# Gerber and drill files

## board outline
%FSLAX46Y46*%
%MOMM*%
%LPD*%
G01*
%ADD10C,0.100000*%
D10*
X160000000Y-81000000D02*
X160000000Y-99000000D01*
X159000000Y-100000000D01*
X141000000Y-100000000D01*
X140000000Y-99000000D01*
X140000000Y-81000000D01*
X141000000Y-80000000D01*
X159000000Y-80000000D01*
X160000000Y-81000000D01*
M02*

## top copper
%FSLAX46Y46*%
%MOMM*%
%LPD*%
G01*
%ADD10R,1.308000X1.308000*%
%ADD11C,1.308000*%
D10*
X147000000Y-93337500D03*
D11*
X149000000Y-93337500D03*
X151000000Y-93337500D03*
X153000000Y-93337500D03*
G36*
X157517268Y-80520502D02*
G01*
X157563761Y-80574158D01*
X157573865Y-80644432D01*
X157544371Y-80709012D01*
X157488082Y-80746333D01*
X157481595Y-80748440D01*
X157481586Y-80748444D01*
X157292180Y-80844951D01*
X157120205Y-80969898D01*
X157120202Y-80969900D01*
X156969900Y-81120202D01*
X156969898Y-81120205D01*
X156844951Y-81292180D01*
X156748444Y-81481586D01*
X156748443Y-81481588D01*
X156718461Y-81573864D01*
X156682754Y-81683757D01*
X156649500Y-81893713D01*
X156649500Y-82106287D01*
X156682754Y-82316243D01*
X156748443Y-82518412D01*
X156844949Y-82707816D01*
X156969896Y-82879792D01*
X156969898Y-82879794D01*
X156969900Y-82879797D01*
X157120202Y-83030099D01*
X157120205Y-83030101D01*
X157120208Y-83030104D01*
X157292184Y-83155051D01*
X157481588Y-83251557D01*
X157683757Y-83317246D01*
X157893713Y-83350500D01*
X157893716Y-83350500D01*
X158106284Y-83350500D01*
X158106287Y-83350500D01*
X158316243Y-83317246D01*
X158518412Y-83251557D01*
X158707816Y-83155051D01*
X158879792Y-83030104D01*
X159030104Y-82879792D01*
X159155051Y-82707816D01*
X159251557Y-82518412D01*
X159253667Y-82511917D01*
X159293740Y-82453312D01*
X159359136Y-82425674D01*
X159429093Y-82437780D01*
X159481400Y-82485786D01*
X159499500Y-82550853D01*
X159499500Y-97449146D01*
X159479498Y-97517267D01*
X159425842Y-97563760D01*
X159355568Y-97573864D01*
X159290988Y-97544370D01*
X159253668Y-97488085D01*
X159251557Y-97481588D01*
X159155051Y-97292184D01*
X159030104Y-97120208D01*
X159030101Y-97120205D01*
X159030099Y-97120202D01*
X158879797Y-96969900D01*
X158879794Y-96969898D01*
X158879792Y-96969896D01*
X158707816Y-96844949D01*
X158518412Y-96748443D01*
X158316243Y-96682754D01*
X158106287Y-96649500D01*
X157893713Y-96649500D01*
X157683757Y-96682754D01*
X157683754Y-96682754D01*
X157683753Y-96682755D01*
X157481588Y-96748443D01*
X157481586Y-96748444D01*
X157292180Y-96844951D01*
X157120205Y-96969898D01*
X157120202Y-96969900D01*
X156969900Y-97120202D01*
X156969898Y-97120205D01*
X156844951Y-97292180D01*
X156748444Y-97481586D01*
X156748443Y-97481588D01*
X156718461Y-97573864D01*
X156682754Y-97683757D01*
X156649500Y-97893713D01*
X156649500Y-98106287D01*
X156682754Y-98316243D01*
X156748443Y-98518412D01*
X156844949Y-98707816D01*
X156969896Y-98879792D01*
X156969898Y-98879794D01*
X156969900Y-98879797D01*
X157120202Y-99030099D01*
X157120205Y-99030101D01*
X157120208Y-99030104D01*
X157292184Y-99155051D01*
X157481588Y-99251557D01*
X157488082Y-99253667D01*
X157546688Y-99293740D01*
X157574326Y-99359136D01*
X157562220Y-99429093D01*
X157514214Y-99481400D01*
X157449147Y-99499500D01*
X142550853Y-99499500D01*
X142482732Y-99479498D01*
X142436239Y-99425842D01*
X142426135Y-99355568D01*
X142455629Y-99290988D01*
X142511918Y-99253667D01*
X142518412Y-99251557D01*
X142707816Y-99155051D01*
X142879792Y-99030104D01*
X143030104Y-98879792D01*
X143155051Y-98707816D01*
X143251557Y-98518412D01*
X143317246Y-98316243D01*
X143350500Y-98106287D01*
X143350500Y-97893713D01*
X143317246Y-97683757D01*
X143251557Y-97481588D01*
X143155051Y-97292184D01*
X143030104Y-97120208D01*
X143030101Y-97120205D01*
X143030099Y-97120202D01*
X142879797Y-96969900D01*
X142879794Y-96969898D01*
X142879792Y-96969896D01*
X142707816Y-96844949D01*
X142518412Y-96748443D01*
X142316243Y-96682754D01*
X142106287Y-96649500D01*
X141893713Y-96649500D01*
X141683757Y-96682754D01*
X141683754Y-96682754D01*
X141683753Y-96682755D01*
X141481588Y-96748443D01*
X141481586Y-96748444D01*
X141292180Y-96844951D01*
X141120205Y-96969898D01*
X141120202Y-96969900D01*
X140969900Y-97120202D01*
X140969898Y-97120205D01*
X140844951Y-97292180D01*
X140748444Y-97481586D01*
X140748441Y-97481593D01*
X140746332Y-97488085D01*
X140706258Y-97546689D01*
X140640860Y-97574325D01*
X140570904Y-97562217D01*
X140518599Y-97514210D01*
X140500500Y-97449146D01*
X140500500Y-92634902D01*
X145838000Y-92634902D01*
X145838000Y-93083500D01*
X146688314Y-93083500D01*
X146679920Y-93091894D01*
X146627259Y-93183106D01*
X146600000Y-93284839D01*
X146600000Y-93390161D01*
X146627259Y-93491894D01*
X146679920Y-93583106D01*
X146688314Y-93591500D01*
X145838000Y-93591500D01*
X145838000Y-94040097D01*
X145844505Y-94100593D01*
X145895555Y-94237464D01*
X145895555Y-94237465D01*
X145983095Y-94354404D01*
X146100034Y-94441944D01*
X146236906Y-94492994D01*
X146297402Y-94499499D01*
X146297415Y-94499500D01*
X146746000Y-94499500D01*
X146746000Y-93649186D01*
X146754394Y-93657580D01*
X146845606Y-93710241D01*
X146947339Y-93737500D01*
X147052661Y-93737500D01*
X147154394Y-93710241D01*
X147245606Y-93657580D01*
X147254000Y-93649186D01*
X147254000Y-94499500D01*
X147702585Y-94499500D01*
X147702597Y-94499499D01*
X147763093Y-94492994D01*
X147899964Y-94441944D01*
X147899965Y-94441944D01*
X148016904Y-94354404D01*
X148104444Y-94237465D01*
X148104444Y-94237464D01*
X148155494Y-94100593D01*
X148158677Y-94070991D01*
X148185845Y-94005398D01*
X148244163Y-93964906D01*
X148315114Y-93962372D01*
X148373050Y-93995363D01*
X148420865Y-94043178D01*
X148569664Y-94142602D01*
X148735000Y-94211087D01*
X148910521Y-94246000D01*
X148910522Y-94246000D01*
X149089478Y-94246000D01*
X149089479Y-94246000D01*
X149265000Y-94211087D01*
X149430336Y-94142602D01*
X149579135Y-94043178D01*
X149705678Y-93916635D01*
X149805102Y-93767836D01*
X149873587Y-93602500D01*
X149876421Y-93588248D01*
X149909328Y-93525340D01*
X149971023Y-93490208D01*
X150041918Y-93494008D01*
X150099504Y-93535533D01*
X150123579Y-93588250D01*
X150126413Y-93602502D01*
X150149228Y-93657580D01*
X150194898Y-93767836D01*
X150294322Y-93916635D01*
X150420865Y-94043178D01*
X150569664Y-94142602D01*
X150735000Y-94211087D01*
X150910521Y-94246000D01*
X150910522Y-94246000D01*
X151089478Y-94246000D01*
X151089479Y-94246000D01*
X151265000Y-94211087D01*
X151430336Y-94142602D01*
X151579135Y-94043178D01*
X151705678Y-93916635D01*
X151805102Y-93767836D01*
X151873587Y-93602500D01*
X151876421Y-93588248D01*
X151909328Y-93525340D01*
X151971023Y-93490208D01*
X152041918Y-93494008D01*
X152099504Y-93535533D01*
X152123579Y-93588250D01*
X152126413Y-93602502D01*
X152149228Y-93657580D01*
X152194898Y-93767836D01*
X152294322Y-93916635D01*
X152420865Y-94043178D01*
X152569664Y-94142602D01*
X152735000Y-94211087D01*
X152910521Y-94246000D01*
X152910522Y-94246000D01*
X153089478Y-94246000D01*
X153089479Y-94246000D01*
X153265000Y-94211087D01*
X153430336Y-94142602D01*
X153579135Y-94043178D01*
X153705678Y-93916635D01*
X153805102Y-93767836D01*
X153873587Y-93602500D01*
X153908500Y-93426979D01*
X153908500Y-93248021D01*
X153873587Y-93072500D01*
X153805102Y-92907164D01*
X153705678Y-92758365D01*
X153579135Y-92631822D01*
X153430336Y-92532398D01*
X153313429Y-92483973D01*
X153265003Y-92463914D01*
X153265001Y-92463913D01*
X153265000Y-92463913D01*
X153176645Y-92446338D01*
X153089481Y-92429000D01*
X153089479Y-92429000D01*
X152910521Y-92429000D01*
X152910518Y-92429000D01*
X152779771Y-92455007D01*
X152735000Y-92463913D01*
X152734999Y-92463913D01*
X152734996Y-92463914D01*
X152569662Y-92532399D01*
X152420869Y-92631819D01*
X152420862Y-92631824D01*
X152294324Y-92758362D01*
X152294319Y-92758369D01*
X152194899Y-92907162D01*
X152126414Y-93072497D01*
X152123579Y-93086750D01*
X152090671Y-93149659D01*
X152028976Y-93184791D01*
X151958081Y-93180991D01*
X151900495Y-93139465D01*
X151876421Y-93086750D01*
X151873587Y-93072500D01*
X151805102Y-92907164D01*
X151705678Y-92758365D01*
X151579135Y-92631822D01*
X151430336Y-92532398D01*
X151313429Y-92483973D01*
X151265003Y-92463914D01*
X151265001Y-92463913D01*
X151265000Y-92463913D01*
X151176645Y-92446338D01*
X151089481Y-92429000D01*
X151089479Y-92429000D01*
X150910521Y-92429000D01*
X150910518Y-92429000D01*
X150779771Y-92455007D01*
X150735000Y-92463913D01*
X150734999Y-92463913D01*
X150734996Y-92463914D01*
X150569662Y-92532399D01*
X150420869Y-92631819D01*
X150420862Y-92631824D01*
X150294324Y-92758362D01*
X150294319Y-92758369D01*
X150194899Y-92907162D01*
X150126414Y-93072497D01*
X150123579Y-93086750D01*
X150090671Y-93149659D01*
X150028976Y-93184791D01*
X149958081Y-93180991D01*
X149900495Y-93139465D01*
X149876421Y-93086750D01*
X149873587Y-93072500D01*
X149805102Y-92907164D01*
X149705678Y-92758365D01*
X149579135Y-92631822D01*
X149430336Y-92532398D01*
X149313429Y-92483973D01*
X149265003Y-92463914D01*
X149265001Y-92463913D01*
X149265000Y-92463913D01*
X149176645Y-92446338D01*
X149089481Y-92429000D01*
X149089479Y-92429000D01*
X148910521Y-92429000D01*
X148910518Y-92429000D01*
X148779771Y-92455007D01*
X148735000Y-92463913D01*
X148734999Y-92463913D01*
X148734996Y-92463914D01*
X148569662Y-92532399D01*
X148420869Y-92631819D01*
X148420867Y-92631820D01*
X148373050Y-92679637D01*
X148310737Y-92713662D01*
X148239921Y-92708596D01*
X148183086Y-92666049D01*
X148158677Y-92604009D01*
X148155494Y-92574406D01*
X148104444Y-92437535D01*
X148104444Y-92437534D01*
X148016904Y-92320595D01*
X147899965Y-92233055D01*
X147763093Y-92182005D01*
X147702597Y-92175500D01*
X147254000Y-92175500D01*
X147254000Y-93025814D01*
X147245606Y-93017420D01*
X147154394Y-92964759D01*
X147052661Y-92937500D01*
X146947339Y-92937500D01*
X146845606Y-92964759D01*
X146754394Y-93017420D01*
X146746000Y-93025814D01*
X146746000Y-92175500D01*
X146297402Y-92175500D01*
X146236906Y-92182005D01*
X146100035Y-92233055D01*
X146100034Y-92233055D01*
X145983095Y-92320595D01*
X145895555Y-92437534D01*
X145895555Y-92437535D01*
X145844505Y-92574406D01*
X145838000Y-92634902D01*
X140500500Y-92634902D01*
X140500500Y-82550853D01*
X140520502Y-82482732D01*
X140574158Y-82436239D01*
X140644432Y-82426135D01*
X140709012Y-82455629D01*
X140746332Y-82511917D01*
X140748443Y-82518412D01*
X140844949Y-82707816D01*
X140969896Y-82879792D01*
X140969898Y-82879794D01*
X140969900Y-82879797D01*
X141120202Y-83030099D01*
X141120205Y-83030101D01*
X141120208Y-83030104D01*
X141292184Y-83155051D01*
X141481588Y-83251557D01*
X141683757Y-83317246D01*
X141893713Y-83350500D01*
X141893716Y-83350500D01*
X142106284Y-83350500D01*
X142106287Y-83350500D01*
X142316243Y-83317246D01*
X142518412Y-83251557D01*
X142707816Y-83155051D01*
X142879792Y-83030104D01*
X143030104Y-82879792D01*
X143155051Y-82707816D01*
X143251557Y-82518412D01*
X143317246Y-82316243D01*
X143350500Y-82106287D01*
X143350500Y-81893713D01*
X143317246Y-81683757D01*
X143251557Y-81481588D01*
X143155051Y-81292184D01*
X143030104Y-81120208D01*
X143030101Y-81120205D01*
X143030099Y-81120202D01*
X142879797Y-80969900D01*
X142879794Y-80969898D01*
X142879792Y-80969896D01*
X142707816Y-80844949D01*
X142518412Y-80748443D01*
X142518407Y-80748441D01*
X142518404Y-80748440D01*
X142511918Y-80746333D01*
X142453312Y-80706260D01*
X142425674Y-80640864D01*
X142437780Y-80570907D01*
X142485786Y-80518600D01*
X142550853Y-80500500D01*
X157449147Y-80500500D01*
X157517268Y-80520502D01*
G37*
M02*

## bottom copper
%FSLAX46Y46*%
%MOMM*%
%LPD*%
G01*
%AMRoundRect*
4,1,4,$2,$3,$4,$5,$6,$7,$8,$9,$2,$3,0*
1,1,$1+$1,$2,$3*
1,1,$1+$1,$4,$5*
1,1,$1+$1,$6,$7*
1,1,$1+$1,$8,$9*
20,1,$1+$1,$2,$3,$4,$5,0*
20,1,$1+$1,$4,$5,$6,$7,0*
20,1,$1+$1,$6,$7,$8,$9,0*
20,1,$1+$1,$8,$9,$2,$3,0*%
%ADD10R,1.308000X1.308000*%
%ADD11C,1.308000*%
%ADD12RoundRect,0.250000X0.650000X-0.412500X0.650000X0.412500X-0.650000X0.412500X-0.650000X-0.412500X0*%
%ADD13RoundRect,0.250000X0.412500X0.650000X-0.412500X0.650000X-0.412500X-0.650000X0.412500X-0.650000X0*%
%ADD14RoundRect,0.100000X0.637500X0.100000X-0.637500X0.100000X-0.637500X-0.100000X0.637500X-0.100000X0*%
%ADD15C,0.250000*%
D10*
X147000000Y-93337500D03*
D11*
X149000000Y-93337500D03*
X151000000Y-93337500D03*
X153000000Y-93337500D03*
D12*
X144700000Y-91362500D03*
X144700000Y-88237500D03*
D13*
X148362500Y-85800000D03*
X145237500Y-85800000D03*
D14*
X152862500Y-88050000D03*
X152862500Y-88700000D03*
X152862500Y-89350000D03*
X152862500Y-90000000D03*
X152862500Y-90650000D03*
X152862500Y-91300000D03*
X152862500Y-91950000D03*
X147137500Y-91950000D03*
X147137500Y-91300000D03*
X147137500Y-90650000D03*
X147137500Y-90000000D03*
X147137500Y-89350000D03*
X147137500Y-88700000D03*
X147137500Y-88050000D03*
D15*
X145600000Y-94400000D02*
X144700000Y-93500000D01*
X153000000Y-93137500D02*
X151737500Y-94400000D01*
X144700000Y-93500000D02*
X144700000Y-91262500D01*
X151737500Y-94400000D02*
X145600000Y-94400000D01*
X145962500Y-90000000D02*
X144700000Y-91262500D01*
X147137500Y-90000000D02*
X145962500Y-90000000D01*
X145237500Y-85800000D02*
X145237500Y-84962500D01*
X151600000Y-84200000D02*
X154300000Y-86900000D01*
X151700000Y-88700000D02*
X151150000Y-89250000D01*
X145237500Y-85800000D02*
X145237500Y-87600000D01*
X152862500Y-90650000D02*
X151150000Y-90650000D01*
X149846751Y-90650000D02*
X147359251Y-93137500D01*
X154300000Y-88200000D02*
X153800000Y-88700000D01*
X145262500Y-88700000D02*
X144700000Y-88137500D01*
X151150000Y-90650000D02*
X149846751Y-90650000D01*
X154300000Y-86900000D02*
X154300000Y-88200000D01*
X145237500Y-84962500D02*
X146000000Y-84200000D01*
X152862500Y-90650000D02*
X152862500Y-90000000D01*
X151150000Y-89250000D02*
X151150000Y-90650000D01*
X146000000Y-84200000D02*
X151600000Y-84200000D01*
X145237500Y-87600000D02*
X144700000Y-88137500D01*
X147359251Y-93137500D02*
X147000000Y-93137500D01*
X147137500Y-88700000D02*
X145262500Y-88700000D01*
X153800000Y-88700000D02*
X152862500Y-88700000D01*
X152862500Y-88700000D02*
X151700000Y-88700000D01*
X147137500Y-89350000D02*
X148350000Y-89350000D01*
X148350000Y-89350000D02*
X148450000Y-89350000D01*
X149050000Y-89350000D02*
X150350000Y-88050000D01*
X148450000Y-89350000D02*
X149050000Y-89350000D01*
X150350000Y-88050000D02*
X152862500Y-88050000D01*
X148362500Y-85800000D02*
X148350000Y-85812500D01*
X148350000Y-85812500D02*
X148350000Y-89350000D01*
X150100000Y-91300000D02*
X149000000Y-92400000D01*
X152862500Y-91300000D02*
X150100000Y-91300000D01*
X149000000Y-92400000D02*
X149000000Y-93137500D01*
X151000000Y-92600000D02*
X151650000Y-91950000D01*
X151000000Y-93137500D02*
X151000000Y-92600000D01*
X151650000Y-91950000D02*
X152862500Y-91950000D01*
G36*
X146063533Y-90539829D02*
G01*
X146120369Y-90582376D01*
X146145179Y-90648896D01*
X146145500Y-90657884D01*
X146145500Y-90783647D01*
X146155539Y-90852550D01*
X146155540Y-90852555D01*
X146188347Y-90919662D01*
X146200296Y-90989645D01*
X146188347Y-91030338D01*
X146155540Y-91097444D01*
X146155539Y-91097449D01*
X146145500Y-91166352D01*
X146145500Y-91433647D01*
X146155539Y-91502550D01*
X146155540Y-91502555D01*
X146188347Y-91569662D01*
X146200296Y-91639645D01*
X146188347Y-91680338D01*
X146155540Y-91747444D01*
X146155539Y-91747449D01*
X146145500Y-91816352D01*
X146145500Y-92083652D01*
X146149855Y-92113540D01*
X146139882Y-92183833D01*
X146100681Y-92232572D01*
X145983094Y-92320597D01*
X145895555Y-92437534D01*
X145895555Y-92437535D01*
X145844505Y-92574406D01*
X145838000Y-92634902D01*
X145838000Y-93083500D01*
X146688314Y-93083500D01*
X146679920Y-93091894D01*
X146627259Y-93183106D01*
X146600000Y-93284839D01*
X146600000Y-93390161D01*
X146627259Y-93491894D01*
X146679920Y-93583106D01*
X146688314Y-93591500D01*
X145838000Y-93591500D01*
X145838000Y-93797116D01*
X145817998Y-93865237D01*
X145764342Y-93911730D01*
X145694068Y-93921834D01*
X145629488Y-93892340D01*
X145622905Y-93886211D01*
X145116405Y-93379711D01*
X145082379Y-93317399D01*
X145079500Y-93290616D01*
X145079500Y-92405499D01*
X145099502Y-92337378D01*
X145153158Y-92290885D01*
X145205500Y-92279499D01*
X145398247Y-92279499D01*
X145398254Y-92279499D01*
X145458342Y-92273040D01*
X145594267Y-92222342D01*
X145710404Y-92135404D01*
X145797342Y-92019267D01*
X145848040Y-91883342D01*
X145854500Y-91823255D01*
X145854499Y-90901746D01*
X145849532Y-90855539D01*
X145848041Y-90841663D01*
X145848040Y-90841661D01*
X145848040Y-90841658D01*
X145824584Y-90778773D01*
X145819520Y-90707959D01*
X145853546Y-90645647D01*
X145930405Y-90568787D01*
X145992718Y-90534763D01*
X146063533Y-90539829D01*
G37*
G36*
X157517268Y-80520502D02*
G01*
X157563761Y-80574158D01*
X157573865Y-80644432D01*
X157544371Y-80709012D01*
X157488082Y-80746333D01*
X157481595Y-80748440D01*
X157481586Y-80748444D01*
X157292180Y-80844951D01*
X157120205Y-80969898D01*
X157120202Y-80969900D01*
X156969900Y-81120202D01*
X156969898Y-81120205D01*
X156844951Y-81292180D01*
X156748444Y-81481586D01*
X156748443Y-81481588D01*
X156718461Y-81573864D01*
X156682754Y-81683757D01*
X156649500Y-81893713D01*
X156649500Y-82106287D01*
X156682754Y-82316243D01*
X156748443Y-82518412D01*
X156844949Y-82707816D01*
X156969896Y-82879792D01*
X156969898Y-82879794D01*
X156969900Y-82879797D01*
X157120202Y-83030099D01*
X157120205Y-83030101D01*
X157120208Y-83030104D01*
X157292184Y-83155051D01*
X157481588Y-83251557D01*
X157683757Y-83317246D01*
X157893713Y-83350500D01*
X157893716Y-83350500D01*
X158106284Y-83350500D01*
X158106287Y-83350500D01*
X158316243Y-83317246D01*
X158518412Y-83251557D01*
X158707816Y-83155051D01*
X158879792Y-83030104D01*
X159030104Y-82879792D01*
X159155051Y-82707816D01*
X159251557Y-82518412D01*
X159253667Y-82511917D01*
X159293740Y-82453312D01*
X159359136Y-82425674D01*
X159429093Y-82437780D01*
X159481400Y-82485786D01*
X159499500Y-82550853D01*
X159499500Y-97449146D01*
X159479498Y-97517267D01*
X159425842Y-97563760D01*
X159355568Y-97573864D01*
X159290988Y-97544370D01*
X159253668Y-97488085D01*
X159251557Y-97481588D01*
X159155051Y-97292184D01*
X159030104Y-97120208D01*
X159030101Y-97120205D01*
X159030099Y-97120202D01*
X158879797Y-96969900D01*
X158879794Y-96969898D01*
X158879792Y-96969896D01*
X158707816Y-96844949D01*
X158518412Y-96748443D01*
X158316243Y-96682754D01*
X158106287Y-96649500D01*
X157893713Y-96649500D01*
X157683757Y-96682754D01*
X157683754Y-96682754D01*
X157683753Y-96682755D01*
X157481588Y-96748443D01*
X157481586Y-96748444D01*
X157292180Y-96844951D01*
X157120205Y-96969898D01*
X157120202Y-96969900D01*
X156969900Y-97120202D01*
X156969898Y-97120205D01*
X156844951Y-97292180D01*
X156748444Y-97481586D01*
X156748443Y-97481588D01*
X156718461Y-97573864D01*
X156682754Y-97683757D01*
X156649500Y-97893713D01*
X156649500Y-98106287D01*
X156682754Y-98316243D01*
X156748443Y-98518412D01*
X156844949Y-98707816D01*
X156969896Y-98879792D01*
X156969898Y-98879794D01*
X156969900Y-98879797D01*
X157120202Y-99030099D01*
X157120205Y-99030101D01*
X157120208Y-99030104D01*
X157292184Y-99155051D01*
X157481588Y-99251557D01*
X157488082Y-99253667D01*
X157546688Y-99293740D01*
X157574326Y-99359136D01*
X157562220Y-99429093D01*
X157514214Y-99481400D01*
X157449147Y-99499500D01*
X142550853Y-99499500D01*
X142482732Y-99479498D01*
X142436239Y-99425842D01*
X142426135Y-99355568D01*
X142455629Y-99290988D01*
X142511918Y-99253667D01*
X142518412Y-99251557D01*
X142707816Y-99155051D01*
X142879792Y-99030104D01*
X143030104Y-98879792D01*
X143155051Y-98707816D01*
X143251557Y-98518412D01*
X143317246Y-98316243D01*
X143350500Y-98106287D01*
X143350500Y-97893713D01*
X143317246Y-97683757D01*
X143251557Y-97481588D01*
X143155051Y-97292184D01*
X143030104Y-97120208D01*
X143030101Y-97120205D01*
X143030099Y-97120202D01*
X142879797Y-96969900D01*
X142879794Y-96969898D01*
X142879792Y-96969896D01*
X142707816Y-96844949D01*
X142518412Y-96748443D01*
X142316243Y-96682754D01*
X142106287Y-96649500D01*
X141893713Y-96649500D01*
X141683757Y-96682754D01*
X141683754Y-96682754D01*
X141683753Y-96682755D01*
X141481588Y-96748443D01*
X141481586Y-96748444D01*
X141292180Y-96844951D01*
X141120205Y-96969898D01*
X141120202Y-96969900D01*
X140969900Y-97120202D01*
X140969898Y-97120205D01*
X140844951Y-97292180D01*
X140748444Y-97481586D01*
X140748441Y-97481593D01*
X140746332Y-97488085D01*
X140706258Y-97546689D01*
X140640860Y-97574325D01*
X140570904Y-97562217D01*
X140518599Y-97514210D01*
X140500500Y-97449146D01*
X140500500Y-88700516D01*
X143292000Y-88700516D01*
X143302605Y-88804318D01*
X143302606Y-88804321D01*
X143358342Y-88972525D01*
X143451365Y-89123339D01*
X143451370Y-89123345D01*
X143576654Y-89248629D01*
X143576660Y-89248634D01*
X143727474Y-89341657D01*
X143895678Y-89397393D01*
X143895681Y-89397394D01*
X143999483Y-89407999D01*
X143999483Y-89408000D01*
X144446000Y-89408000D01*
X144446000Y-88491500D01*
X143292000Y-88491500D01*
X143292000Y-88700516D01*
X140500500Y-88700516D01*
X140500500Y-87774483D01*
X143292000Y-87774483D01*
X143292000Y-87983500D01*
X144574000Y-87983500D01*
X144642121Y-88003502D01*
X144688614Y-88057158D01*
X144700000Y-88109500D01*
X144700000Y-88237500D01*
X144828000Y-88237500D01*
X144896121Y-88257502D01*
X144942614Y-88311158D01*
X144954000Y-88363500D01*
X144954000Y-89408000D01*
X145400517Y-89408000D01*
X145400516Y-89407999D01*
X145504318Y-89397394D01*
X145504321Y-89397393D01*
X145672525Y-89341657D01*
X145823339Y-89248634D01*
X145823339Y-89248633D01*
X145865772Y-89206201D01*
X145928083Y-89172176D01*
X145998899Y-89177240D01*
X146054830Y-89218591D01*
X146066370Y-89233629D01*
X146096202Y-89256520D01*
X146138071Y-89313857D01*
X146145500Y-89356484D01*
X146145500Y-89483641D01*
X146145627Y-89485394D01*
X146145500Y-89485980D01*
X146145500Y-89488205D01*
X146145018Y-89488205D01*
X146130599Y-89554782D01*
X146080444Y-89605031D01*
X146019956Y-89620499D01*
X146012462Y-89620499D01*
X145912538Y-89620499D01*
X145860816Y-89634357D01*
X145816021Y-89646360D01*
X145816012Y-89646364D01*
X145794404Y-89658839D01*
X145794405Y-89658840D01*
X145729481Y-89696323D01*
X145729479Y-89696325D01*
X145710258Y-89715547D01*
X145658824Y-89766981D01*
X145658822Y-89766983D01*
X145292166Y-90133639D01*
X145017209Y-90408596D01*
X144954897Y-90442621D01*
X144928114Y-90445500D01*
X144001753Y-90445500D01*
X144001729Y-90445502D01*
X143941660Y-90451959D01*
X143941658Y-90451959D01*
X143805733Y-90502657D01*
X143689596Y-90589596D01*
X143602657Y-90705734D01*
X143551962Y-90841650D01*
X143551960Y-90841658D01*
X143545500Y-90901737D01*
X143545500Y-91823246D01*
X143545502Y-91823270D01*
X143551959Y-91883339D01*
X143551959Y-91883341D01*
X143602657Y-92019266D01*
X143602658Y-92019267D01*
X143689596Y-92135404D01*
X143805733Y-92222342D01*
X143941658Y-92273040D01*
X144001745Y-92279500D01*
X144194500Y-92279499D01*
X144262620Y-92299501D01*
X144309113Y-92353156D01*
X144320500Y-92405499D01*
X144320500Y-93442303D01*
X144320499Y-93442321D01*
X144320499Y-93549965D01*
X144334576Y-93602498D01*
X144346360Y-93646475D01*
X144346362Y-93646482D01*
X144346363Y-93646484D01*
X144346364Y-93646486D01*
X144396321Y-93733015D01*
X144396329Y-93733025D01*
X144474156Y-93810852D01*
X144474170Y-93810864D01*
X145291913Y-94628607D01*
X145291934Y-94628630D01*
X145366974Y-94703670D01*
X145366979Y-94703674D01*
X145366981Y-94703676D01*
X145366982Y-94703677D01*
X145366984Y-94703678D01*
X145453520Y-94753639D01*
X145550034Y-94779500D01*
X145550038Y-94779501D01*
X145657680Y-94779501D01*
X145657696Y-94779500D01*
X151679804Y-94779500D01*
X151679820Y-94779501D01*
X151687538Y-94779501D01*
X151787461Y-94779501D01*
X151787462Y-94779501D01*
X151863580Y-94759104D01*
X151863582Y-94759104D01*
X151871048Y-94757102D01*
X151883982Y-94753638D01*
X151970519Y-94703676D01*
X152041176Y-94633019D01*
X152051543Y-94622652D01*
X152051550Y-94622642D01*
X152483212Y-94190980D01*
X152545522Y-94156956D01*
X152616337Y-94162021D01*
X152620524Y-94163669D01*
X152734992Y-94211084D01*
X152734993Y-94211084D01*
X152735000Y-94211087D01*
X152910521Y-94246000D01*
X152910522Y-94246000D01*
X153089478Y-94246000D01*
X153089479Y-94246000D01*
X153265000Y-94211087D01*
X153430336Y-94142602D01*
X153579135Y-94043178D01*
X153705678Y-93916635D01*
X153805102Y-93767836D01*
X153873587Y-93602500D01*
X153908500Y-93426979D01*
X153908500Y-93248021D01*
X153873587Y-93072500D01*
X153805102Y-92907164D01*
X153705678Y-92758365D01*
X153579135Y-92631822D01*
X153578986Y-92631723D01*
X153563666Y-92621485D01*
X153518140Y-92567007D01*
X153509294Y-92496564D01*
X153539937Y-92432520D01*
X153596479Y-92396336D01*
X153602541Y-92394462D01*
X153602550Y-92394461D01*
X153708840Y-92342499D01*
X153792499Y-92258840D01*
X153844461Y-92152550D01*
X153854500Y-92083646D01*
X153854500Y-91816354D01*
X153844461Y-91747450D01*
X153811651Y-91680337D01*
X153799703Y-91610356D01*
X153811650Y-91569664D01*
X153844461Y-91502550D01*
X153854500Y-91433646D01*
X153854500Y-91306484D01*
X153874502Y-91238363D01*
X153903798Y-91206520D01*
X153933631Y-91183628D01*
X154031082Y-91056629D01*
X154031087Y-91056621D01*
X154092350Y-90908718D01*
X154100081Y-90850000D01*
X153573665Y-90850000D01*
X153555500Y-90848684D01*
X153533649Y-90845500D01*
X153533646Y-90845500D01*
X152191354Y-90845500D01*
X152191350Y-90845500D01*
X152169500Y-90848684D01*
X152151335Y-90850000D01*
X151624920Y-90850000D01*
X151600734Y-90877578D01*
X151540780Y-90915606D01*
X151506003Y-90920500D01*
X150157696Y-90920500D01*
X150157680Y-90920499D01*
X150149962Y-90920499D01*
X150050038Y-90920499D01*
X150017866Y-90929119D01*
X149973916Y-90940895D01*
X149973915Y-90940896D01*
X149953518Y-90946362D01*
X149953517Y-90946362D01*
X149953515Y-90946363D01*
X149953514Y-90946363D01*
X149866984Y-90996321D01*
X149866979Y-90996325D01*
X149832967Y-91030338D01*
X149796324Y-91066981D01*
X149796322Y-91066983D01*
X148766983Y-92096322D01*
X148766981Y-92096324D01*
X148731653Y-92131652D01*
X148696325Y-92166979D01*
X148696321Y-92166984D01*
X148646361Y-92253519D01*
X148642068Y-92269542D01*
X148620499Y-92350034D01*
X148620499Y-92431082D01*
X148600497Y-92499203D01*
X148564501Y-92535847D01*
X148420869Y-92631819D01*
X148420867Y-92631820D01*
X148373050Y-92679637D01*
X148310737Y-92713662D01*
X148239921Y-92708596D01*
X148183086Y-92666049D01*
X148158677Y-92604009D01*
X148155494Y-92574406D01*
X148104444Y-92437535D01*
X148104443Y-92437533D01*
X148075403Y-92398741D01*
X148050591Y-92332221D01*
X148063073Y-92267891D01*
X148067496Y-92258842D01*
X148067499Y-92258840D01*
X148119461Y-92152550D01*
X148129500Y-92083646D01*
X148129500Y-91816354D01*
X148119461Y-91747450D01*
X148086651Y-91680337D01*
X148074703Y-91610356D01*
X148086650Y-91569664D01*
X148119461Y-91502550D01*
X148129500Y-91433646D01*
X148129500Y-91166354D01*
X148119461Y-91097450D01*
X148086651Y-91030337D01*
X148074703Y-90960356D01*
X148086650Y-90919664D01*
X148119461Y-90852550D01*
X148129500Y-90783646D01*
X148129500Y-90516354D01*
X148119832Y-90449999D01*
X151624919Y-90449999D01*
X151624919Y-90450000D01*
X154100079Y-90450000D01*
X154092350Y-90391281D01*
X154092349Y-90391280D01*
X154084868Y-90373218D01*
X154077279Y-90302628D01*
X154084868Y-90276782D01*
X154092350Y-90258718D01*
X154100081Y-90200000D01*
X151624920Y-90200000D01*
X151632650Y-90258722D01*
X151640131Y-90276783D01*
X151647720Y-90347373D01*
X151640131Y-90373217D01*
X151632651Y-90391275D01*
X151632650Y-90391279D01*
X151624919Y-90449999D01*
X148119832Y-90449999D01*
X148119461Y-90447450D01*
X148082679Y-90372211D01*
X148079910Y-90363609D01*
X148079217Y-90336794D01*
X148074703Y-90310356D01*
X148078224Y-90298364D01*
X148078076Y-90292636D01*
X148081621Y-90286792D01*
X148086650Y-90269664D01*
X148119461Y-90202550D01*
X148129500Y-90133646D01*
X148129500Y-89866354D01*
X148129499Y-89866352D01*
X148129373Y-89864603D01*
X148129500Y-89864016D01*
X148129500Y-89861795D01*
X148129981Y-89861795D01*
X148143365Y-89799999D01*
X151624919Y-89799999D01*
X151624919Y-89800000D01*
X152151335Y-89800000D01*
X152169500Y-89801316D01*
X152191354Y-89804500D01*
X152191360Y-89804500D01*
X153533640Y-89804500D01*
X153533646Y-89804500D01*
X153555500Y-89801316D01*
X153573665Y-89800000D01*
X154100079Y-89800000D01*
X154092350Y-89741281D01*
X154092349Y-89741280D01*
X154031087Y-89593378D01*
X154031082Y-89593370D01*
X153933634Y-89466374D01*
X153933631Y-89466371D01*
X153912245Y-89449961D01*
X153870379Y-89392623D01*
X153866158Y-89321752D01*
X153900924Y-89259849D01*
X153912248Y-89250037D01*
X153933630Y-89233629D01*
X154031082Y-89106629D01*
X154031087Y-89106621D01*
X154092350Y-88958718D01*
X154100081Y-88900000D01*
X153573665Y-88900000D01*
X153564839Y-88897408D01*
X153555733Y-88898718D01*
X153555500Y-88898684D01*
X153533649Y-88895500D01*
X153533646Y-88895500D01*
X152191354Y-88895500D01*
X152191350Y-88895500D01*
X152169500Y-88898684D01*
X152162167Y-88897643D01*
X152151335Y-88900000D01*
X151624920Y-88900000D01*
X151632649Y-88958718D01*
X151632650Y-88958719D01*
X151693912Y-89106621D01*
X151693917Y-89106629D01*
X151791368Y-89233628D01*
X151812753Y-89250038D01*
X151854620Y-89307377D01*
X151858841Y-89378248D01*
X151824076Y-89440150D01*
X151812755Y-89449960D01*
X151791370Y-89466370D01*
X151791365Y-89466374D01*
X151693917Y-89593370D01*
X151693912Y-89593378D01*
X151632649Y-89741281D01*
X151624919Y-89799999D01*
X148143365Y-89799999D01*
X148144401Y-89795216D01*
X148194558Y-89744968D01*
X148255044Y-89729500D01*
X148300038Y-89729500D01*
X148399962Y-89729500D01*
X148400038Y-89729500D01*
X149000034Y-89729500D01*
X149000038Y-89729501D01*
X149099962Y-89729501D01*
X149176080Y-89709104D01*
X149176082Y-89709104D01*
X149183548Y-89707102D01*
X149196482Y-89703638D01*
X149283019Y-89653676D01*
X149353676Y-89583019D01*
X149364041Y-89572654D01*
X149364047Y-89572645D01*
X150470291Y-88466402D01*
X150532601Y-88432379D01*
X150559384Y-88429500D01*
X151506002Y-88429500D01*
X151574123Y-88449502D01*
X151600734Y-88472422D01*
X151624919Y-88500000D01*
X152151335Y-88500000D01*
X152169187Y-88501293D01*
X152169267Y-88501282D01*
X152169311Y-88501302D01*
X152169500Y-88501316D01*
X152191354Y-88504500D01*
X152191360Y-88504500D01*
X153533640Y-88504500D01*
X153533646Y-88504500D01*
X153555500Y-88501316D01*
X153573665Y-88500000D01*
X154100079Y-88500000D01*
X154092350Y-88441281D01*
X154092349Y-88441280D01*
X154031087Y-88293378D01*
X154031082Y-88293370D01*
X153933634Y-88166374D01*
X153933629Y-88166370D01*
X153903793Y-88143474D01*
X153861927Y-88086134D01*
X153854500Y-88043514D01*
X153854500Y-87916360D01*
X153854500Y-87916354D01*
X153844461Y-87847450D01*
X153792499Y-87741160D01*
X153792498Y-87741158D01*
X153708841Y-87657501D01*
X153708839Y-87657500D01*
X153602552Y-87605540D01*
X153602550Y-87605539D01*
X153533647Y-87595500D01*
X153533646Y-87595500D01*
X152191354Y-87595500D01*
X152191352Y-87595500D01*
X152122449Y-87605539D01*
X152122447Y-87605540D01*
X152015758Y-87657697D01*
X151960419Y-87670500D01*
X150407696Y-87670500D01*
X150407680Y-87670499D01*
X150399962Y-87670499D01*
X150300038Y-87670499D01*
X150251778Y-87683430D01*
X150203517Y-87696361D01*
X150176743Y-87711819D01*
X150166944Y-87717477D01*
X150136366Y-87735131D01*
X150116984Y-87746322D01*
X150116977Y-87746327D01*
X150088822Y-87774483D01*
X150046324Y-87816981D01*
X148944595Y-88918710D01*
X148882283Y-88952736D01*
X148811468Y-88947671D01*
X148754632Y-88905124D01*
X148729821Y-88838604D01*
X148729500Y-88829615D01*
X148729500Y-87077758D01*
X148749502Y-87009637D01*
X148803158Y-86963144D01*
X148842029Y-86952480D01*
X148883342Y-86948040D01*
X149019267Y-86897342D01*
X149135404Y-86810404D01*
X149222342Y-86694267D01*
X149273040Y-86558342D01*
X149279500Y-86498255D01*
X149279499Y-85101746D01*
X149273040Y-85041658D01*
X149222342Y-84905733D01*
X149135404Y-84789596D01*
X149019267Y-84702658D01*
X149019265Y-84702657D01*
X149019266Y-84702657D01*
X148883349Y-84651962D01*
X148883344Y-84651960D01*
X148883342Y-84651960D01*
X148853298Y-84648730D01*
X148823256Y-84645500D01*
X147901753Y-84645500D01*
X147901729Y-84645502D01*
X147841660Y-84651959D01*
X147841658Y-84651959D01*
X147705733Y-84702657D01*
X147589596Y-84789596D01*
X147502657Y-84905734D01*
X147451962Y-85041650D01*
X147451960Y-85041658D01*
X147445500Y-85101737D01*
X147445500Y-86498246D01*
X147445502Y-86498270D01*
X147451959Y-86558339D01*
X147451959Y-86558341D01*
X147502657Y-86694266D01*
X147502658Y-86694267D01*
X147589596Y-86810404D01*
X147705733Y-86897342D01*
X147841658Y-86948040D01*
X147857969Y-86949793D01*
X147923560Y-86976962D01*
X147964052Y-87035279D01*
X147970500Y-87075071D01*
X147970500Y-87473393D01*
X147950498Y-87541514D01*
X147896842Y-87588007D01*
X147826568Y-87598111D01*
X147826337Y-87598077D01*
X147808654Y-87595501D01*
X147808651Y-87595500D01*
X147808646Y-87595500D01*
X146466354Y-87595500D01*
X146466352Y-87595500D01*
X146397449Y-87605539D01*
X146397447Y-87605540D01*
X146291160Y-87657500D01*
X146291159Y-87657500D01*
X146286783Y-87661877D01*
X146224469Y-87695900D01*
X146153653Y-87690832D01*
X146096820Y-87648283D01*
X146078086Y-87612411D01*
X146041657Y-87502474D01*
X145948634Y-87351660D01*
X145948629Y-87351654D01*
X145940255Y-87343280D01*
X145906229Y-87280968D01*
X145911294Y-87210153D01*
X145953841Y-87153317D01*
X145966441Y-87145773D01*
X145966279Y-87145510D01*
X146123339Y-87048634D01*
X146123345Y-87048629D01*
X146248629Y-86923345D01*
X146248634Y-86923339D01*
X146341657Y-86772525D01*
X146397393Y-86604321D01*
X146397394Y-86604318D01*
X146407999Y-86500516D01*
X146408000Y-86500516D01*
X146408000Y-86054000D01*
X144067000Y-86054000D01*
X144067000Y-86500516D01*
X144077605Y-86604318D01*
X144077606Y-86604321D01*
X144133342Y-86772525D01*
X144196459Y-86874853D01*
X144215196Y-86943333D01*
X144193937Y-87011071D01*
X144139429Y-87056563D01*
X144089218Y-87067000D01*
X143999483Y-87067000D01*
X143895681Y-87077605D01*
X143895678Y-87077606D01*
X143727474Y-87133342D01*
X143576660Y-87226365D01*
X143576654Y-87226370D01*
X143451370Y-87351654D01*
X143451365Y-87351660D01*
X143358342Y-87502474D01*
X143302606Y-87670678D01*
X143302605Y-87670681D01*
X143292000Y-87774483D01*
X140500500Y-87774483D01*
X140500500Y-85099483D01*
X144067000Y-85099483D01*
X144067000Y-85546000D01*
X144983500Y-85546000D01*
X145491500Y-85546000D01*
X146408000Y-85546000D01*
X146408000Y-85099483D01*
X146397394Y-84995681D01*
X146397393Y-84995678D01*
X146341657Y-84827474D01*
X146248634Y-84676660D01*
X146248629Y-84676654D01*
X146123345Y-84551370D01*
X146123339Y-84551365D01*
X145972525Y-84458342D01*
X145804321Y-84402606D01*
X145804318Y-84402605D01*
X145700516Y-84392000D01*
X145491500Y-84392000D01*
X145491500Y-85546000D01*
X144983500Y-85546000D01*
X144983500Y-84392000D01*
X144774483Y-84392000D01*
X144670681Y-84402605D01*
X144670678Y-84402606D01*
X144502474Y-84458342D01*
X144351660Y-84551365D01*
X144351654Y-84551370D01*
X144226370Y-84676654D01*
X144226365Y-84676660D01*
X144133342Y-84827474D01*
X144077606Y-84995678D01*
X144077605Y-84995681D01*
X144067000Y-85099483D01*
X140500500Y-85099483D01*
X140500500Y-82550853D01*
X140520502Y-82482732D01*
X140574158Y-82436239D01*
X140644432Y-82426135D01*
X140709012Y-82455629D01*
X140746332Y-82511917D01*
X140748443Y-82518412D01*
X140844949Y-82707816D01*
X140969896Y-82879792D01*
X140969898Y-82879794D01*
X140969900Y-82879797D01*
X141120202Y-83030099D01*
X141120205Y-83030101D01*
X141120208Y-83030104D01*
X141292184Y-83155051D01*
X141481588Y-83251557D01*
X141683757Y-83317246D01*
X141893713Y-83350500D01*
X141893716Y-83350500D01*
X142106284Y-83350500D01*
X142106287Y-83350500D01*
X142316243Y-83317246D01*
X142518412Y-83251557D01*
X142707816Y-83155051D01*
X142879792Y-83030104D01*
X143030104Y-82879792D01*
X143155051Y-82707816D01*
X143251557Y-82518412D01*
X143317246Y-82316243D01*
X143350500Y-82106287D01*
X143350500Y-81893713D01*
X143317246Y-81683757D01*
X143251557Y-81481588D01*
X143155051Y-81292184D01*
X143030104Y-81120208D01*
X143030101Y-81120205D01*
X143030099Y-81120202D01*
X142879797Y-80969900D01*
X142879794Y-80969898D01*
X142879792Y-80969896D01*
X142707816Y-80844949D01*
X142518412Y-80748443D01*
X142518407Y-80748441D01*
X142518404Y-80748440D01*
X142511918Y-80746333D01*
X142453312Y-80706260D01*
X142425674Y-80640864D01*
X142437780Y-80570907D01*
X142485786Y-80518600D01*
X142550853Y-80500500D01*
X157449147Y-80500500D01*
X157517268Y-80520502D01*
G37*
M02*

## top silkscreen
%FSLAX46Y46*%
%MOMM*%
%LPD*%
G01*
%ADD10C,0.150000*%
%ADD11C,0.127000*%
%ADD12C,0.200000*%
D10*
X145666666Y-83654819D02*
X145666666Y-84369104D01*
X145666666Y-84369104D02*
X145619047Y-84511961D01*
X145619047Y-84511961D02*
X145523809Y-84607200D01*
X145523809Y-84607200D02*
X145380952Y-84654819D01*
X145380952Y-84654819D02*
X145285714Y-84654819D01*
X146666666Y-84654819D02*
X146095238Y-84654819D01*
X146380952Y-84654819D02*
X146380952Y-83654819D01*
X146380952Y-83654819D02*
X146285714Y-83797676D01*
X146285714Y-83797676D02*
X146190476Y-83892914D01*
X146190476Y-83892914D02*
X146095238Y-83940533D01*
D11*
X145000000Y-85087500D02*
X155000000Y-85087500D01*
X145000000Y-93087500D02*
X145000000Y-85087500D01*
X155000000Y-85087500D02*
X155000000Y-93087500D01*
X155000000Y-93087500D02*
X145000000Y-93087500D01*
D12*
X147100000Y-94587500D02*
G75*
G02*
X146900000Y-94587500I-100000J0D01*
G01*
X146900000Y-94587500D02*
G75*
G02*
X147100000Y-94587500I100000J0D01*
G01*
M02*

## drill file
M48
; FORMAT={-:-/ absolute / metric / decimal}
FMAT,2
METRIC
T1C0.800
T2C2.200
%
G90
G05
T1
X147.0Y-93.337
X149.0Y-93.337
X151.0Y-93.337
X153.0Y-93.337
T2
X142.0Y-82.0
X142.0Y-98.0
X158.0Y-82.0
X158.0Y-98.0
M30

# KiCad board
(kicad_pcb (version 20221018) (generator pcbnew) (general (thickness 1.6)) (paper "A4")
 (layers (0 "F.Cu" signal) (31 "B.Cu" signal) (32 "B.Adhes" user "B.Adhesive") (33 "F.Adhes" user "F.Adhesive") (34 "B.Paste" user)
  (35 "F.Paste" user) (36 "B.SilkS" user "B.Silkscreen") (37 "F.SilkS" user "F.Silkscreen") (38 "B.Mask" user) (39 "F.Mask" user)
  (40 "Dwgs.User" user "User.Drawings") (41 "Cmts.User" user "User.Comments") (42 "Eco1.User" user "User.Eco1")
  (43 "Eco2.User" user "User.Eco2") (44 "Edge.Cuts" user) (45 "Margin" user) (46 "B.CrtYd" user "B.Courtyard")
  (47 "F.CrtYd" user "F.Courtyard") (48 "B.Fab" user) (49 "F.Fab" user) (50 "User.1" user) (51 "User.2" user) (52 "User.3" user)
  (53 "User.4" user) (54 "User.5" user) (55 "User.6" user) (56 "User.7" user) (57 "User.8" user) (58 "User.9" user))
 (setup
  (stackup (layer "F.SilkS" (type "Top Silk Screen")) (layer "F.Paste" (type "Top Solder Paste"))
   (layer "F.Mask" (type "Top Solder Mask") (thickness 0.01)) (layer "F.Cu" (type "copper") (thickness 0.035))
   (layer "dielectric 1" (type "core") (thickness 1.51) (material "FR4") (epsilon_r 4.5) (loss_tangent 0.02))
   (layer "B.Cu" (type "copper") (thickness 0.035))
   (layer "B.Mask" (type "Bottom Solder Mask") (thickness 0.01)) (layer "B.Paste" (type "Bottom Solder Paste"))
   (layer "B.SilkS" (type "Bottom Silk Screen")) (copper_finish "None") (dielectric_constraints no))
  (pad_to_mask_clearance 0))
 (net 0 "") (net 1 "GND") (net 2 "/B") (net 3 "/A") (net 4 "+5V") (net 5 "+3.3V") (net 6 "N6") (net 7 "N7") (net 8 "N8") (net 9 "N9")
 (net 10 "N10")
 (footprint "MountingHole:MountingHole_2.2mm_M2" (layer "F.Cu") (at 142 82)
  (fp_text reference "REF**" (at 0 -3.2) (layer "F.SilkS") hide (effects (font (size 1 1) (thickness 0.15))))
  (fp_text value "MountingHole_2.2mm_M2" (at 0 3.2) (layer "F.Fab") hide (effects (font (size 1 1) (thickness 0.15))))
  (pad "" np_thru_hole circle (at 0 0) (size 2.2 2.2) (drill 2.2) (layers "F&B.Cu" "*.Mask")))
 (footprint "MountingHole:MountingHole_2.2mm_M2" (layer "F.Cu") (at 158 98)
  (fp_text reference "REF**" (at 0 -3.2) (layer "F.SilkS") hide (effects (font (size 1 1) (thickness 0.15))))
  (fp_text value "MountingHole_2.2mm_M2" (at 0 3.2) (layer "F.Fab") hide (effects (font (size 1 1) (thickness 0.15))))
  (pad "" np_thru_hole circle (at 0 0) (size 2.2 2.2) (drill 2.2) (layers "F&B.Cu" "*.Mask")))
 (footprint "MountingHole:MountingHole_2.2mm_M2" (layer "F.Cu") (at 142 98)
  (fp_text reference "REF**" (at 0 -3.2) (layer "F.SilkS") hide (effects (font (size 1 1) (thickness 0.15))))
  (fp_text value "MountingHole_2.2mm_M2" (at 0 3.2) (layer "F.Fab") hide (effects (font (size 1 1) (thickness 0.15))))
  (pad "" np_thru_hole circle (at 0 0) (size 2.2 2.2) (drill 2.2) (layers "*.Cu" "*.Mask")))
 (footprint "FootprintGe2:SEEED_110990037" (layer "F.Cu") (at 150 93.3375)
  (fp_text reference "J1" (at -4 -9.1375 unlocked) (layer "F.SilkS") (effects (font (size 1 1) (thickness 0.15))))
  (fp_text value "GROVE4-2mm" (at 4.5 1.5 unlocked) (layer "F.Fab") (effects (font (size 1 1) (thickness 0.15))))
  (fp_line (start -5 -8.25) (end 5 -8.25) (stroke (width 0.127) (type solid)) (layer "F.SilkS"))
  (fp_line (start -5 -0.25) (end -5 -8.25) (stroke (width 0.127) (type solid)) (layer "F.SilkS"))
  (fp_line (start 5 -8.25) (end 5 -0.25) (stroke (width 0.127) (type solid)) (layer "F.SilkS"))
  (fp_line (start 5 -0.25) (end -5 -0.25) (stroke (width 0.127) (type solid)) (layer "F.SilkS"))
  (fp_circle (center -3 1.25) (end -2.9 1.25) (stroke (width 0.2) (type solid)) (fill none) (layer "F.SilkS"))
  (pad "1" thru_hole rect (at -3 0) (size 1.308 1.308) (drill 0.8) (layers "*.Cu" "*.Mask") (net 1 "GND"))
  (pad "2" thru_hole circle (at -1 0) (size 1.308 1.308) (drill 0.8) (layers "*.Cu" "*.Mask") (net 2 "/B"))
  (pad "3" thru_hole circle (at 1 0) (size 1.308 1.308) (drill 0.8) (layers "*.Cu" "*.Mask") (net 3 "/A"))
  (pad "4" thru_hole circle (at 3 0) (size 1.308 1.308) (drill 0.8) (layers "*.Cu" "*.Mask") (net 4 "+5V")))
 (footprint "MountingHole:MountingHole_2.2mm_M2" (layer "F.Cu") (at 158 82)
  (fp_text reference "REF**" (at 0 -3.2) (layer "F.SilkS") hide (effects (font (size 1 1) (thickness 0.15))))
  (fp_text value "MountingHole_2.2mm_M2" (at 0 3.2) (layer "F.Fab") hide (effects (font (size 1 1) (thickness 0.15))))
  (pad "" np_thru_hole circle (at 0 0) (size 2.2 2.2) (drill 2.2) (layers "F&B.Cu" "*.Mask")))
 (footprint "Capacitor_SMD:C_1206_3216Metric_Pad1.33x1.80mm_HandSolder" (layer "B.Cu") (at 144.7 89.8 90)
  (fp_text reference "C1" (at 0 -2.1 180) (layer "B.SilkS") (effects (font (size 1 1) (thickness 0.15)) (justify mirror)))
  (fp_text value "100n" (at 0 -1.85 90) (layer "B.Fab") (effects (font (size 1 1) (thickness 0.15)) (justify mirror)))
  (pad "1" smd roundrect (at -1.5625 0 90) (size 1.325 1.8) (layers "B.Cu" "B.Paste" "B.Mask") (roundrect_rratio 0.1886792453) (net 4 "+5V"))
  (pad "2" smd roundrect (at 1.5625 0 90) (size 1.325 1.8) (layers "B.Cu" "B.Paste" "B.Mask") (roundrect_rratio 0.1886792453) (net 1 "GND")))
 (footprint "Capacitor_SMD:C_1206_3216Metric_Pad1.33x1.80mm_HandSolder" (layer "B.Cu") (at 146.8 85.8 180)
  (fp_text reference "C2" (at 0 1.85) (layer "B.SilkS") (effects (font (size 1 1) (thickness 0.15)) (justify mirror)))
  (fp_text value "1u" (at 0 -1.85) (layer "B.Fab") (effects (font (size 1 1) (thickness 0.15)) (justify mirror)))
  (pad "1" smd roundrect (at -1.5625 0 180) (size 1.325 1.8) (layers "B.Cu" "B.Paste" "B.Mask") (roundrect_rratio 0.1886792453)
   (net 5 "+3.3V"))
  (pad "2" smd roundrect (at 1.5625 0 180) (size 1.325 1.8) (layers "B.Cu" "B.Paste" "B.Mask") (roundrect_rratio 0.1886792453) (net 1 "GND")))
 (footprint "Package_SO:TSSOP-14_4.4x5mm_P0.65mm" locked (layer "B.Cu") (at 150 90 180)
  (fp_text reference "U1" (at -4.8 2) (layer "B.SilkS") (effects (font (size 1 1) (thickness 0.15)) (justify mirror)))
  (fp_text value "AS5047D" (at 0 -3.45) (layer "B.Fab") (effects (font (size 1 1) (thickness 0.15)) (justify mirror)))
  (pad "1" smd roundrect locked (at -2.8625 1.95 180) (size 1.475 0.4) (layers "B.Cu" "B.Paste" "B.Mask") (roundrect_rratio 0.25)
   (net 5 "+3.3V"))
  (pad "2" smd roundrect locked (at -2.8625 1.3 180) (size 1.475 0.4) (layers "B.Cu" "B.Paste" "B.Mask") (roundrect_rratio 0.25)
   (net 1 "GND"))
  (pad "3" smd roundrect locked (at -2.8625 0.65 180) (size 1.475 0.4) (layers "B.Cu" "B.Paste" "B.Mask") (roundrect_rratio 0.25)
   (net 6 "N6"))
  (pad "4" smd roundrect locked (at -2.8625 0 180) (size 1.475 0.4) (layers "B.Cu" "B.Paste" "B.Mask") (roundrect_rratio 0.25) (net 1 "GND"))
  (pad "5" smd roundrect locked (at -2.8625 -0.65 180) (size 1.475 0.4) (layers "B.Cu" "B.Paste" "B.Mask") (roundrect_rratio 0.25)
   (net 1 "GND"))
  (pad "6" smd roundrect locked (at -2.8625 -1.3 180) (size 1.475 0.4) (layers "B.Cu" "B.Paste" "B.Mask") (roundrect_rratio 0.25)
   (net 2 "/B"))
  (pad "7" smd roundrect locked (at -2.8625 -1.95 180) (size 1.475 0.4) (layers "B.Cu" "B.Paste" "B.Mask") (roundrect_rratio 0.25)
   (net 3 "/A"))
  (pad "8" smd roundrect locked (at 2.8625 -1.95 180) (size 1.475 0.4) (layers "B.Cu" "B.Paste" "B.Mask") (roundrect_rratio 0.25)
   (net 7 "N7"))
  (pad "9" smd roundrect locked (at 2.8625 -1.3 180) (size 1.475 0.4) (layers "B.Cu" "B.Paste" "B.Mask") (roundrect_rratio 0.25)
   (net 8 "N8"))
  (pad "10" smd roundrect locked (at 2.8625 -0.65 180) (size 1.475 0.4) (layers "B.Cu" "B.Paste" "B.Mask") (roundrect_rratio 0.25)
   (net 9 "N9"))
  (pad "11" smd roundrect locked (at 2.8625 0 180) (size 1.475 0.4) (layers "B.Cu" "B.Paste" "B.Mask") (roundrect_rratio 0.25) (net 4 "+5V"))
  (pad "12" smd roundrect locked (at 2.8625 0.65 180) (size 1.475 0.4) (layers "B.Cu" "B.Paste" "B.Mask") (roundrect_rratio 0.25)
   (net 5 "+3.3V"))
  (pad "13" smd roundrect locked (at 2.8625 1.3 180) (size 1.475 0.4) (layers "B.Cu" "B.Paste" "B.Mask") (roundrect_rratio 0.25)
   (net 1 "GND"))
  (pad "14" smd roundrect locked (at 2.8625 1.95 180) (size 1.475 0.4) (layers "B.Cu" "B.Paste" "B.Mask") (roundrect_rratio 0.25)
   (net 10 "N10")))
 (gr_poly
  (pts (xy 160 81) (xy 160 99) (xy 159 100) (xy 141 100) (xy 140 99) (xy 140 81) (xy 141 80) (xy 159 80)) (stroke (width 0.1) (type solid))
  (fill none) (layer "Edge.Cuts"))
 (segment (start 145.6 94.4) (end 144.7 93.5) (width 0.25) (layer "B.Cu") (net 4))
 (segment (start 153 93.1375) (end 151.7375 94.4) (width 0.25) (layer "B.Cu") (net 4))
 (segment (start 144.7 93.5) (end 144.7 91.2625) (width 0.25) (layer "B.Cu") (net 4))
 (segment (start 151.7375 94.4) (end 145.6 94.4) (width 0.25) (layer "B.Cu") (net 4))
 (segment (start 145.9625 90) (end 144.7 91.2625) (width 0.25) (layer "B.Cu") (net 4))
 (segment (start 147.1375 90) (end 145.9625 90) (width 0.25) (layer "B.Cu") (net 4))
 (segment (start 145.2375 85.8) (end 145.2375 84.9625) (width 0.25) (layer "B.Cu") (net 1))
 (segment (start 151.6 84.2) (end 154.3 86.9) (width 0.25) (layer "B.Cu") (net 1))
 (segment (start 151.7 88.7) (end 151.15 89.25) (width 0.25) (layer "B.Cu") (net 1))
 (segment (start 145.2375 85.8) (end 145.2375 87.6) (width 0.25) (layer "B.Cu") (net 1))
 (segment (start 152.8625 90.65) (end 151.15 90.65) (width 0.25) (layer "B.Cu") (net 1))
 (segment (start 149.846751 90.65) (end 147.359251 93.1375) (width 0.25) (layer "B.Cu") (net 1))
 (segment (start 154.3 88.2) (end 153.8 88.7) (width 0.25) (layer "B.Cu") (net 1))
 (segment (start 145.2625 88.7) (end 144.7 88.1375) (width 0.25) (layer "B.Cu") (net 1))
 (segment (start 151.15 90.65) (end 149.846751 90.65) (width 0.25) (layer "B.Cu") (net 1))
 (segment (start 154.3 86.9) (end 154.3 88.2) (width 0.25) (layer "B.Cu") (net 1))
 (segment (start 145.2375 84.9625) (end 146 84.2) (width 0.25) (layer "B.Cu") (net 1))
 (segment (start 152.8625 90.65) (end 152.8625 90) (width 0.25) (layer "B.Cu") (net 1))
 (segment (start 151.15 89.25) (end 151.15 90.65) (width 0.25) (layer "B.Cu") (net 1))
 (segment (start 146 84.2) (end 151.6 84.2) (width 0.25) (layer "B.Cu") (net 1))
 (segment (start 145.2375 87.6) (end 144.7 88.1375) (width 0.25) (layer "B.Cu") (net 1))
 (segment (start 147.359251 93.1375) (end 147 93.1375) (width 0.25) (layer "B.Cu") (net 1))
 (segment (start 147.1375 88.7) (end 145.2625 88.7) (width 0.25) (layer "B.Cu") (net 1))
 (segment (start 153.8 88.7) (end 152.8625 88.7) (width 0.25) (layer "B.Cu") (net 1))
 (segment (start 152.8625 88.7) (end 151.7 88.7) (width 0.25) (layer "B.Cu") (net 1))
 (segment (start 147.1375 89.35) (end 148.35 89.35) (width 0.25) (layer "B.Cu") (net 5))
 (segment (start 148.35 89.35) (end 148.45 89.35) (width 0.25) (layer "B.Cu") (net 5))
 (segment (start 149.05 89.35) (end 150.35 88.05) (width 0.25) (layer "B.Cu") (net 5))
 (segment (start 148.45 89.35) (end 149.05 89.35) (width 0.25) (layer "B.Cu") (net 5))
 (segment (start 150.35 88.05) (end 152.8625 88.05) (width 0.25) (layer "B.Cu") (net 5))
 (segment (start 148.3625 85.8) (end 148.35 85.8125) (width 0.25) (layer "B.Cu") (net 5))
 (segment (start 148.35 85.8125) (end 148.35 89.35) (width 0.25) (layer "B.Cu") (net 5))
 (segment (start 150.1 91.3) (end 149 92.4) (width 0.25) (layer "B.Cu") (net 2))
 (segment (start 152.8625 91.3) (end 150.1 91.3) (width 0.25) (layer "B.Cu") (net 2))
 (segment (start 149 92.4) (end 149 93.1375) (width 0.25) (layer "B.Cu") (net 2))
 (segment (start 151 92.6) (end 151.65 91.95) (width 0.25) (layer "B.Cu") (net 3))
 (segment (start 151 93.1375) (end 151 92.6) (width 0.25) (layer "B.Cu") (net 3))
 (segment (start 151.65 91.95) (end 152.8625 91.95) (width 0.25) (layer "B.Cu") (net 3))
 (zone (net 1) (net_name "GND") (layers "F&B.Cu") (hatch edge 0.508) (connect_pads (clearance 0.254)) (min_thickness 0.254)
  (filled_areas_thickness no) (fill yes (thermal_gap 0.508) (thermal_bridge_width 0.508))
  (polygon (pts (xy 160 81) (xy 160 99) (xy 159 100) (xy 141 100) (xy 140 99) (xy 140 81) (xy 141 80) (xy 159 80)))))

